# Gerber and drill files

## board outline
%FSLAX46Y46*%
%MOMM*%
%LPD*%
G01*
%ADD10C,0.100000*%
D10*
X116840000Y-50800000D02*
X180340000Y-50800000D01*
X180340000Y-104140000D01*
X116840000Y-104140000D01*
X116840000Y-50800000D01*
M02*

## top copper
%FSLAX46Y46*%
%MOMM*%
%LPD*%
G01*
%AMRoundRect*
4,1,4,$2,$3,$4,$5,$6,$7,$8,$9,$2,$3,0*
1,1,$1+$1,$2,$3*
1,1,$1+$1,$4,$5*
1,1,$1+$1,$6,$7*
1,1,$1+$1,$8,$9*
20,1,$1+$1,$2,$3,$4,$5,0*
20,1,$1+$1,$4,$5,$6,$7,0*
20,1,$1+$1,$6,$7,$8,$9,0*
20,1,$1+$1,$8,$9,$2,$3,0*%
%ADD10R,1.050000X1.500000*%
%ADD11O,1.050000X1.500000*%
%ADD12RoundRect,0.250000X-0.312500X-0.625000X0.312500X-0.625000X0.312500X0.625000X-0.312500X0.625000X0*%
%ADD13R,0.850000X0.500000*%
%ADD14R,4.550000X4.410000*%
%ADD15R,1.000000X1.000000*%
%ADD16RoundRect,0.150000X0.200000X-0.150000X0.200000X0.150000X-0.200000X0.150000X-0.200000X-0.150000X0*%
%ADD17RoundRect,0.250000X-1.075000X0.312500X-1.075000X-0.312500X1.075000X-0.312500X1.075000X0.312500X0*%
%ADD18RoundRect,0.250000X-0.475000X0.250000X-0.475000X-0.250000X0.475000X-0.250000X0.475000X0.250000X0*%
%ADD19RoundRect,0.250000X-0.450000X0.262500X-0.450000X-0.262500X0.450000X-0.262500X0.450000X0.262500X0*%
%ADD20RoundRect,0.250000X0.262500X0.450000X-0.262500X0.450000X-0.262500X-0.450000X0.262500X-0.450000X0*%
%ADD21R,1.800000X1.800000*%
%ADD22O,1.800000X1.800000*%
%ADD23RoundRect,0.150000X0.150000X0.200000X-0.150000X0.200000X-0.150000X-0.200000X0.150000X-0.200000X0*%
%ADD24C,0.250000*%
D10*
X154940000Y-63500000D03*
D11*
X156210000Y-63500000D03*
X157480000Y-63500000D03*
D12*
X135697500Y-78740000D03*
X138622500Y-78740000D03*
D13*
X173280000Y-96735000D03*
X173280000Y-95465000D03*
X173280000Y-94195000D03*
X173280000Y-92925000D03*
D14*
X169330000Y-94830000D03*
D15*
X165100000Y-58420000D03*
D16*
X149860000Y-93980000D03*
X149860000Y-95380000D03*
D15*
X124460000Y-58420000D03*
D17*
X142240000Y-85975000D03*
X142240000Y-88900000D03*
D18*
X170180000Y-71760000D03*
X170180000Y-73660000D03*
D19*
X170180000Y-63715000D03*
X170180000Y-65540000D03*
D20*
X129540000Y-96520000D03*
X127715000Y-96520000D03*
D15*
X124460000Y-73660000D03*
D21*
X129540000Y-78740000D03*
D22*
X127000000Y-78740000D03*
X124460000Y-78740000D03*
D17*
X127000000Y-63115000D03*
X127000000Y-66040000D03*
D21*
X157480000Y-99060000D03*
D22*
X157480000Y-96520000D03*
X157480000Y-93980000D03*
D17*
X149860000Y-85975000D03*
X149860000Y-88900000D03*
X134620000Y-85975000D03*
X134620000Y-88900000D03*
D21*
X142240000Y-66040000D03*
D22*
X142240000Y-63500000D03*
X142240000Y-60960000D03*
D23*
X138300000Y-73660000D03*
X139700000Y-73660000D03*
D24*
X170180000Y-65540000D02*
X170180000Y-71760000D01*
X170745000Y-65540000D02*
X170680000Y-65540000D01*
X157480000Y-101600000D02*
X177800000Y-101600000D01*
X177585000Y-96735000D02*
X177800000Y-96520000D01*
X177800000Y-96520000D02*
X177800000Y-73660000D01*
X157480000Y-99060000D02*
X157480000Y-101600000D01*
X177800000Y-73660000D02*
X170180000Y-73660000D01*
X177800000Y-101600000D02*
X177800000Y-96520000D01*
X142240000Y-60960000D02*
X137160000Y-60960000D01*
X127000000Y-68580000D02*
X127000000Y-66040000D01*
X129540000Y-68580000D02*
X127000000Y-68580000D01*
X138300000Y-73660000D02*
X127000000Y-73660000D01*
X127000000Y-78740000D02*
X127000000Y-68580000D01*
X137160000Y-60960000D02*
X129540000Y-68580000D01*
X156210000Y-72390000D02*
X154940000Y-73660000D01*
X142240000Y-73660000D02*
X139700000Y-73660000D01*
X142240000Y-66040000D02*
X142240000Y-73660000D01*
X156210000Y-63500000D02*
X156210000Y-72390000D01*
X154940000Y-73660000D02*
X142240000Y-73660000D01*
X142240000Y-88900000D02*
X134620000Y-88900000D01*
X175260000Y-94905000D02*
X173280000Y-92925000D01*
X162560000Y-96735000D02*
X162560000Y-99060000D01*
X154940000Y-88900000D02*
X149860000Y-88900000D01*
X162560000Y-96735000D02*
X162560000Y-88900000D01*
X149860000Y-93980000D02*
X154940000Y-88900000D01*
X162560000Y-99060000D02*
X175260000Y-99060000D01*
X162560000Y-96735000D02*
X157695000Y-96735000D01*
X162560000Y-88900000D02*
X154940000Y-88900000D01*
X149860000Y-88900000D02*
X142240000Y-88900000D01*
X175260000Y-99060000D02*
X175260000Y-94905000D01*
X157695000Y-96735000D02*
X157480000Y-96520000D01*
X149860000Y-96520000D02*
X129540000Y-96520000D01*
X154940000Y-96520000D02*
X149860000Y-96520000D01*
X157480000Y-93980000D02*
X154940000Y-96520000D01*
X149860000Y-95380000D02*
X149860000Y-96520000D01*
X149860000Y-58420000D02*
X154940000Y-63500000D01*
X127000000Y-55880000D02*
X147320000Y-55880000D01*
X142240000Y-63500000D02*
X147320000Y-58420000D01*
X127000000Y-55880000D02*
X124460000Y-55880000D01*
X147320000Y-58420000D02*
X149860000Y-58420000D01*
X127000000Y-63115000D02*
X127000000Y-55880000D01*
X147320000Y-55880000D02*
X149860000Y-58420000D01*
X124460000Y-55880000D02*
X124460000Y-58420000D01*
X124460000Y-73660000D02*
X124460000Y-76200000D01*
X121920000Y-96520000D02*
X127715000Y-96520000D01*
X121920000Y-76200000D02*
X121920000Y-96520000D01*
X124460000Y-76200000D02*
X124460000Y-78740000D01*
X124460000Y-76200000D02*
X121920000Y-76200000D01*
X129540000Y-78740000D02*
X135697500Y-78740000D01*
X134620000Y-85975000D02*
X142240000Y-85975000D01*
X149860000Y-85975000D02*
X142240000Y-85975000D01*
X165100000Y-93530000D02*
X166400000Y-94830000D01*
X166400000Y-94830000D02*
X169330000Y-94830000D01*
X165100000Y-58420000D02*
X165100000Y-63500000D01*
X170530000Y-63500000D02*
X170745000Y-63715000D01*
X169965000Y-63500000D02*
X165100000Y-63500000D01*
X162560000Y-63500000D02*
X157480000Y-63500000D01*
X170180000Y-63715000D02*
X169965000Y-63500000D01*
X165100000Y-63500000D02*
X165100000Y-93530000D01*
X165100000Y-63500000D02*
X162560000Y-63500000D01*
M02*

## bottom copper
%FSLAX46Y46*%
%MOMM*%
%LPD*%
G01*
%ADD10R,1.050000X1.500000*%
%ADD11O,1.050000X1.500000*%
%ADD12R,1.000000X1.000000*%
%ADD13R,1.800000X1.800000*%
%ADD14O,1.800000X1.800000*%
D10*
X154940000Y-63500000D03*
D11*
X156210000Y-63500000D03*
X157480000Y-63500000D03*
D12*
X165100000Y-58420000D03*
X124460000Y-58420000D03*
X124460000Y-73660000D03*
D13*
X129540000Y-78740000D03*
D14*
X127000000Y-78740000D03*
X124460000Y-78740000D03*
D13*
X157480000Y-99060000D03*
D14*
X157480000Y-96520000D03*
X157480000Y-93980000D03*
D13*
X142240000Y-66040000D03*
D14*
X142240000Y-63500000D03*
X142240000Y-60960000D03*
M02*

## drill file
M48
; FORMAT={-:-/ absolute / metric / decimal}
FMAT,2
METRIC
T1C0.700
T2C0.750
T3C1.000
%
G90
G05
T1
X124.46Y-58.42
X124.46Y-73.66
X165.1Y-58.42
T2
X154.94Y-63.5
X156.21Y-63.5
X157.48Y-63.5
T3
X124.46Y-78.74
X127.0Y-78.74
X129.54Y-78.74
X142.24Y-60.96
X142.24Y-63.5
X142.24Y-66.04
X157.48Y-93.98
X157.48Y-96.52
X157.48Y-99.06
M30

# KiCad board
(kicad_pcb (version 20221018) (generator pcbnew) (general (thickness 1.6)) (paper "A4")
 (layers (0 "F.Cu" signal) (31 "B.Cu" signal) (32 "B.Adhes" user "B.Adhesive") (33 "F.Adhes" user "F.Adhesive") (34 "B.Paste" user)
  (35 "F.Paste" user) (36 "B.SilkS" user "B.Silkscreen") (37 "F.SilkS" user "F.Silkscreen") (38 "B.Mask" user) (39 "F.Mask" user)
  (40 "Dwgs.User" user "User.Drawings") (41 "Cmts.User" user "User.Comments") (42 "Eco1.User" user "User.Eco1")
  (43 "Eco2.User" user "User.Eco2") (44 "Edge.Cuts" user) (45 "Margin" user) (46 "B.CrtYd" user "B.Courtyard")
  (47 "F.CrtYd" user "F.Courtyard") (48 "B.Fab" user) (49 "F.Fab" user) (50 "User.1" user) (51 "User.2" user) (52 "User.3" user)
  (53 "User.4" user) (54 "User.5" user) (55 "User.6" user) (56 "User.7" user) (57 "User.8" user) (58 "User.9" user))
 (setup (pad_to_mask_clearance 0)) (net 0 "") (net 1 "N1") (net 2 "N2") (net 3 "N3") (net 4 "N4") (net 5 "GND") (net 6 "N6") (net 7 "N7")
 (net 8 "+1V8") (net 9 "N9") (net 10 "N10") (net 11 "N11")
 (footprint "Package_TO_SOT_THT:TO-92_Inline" (layer "F.Cu") (at 154.94 63.5)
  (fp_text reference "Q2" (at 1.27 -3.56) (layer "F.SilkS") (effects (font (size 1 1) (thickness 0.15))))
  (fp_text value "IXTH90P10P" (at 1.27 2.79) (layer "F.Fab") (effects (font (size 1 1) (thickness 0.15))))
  (pad "1" thru_hole rect (at 0 0) (size 1.05 1.5) (drill 0.75) (layers "*.Cu" "*.Mask") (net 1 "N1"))
  (pad "2" thru_hole oval (at 1.27 0) (size 1.05 1.5) (drill 0.75) (layers "*.Cu" "*.Mask") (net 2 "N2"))
  (pad "3" thru_hole oval (at 2.54 0) (size 1.05 1.5) (drill 0.75) (layers "*.Cu" "*.Mask") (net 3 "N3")))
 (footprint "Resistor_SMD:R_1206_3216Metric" (layer "F.Cu") (at 137.16 78.74)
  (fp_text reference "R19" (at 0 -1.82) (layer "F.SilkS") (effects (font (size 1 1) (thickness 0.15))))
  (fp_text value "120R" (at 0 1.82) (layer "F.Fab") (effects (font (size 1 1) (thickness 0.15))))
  (pad "1" smd roundrect (at -1.4625 0) (size 1.125 1.75) (layers "F.Cu" "F.Paste" "F.Mask") (roundrect_rratio 0.222222) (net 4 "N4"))
  (pad "2" smd roundrect (at 1.4625 0) (size 1.125 1.75) (layers "F.Cu" "F.Paste" "F.Mask") (roundrect_rratio 0.222222) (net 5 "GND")))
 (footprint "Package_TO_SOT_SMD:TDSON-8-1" (layer "F.Cu") (at 170.38 94.83 180)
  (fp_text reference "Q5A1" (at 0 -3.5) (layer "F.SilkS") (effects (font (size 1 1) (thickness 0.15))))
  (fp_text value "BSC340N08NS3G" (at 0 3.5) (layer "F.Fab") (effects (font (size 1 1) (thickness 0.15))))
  (pad "" smd rect (at -0.2 -0.85 180) (size 1.5 1.5) (layers "F.Paste"))
  (pad "" smd rect (at -0.2 0.85 180) (size 1.5 1.5) (layers "F.Paste"))
  (pad "" smd custom (at 0.65 0 180) (size 3.75 4.41) (layers "F.Mask") (zone_connect 0) (thermal_bridge_angle 45)
   (options (clearance outline) (anchor rect)) (primitives))
  (pad "" smd rect (at 1.5 -0.85 180) (size 1.5 1.5) (layers "F.Paste"))
  (pad "" smd rect (at 1.5 0.85 180) (size 1.5 1.5) (layers "F.Paste"))
  (pad "" smd rect (at 2.905 -1.905 180) (size 0.75 0.5) (layers "F.Paste"))
  (pad "" smd rect (at 2.905 -0.635 180) (size 0.75 0.5) (layers "F.Paste"))
  (pad "" smd rect (at 2.905 0.635 180) (size 0.75 0.5) (layers "F.Paste"))
  (pad "" smd rect (at 2.905 1.905 180) (size 0.75 0.5) (layers "F.Paste"))
  (pad "1" smd rect (at -2.9 -1.905 180) (size 0.85 0.5) (layers "F.Cu" "F.Paste" "F.Mask") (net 5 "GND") (solder_paste_margin -0.05))
  (pad "2" smd rect (at -2.9 -0.635 180) (size 0.85 0.5) (layers "F.Cu" "F.Paste" "F.Mask") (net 5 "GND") (solder_paste_margin -0.05))
  (pad "3" smd rect (at -2.9 0.635 180) (size 0.85 0.5) (layers "F.Cu" "F.Paste" "F.Mask") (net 5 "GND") (solder_paste_margin -0.05))
  (pad "4" smd rect (at -2.9 1.905 180) (size 0.85 0.5) (layers "F.Cu" "F.Paste" "F.Mask") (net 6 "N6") (solder_paste_margin -0.05))
  (pad "5" smd rect (at 1.05 0 180) (size 4.55 4.41) (layers "F.Cu") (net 3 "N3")))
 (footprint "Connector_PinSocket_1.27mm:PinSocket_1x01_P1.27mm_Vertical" (layer "F.Cu") (at 165.1 58.42)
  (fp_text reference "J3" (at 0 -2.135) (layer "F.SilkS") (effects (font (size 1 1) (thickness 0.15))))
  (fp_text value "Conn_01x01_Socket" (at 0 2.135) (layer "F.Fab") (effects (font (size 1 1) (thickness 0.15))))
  (pad "1" thru_hole rect (at 0 0) (size 1 1) (drill 0.7) (layers "*.Cu" "*.Mask") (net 3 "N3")))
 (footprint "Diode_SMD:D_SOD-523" (layer "F.Cu") (at 149.86 94.68 -90)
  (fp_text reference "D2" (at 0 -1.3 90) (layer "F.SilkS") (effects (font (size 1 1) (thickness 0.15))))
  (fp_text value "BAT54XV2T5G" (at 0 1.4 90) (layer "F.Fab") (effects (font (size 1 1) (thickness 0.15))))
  (pad "1" smd roundrect (at -0.7 0 90) (size 0.6 0.7) (layers "F.Cu" "F.Paste" "F.Mask") (roundrect_rratio 0.25) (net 6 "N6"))
  (pad "2" smd roundrect (at 0.7 0 90) (size 0.6 0.7) (layers "F.Cu" "F.Paste" "F.Mask") (roundrect_rratio 0.25) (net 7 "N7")))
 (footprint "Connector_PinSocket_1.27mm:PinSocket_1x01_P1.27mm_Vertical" (layer "F.Cu") (at 124.46 58.42)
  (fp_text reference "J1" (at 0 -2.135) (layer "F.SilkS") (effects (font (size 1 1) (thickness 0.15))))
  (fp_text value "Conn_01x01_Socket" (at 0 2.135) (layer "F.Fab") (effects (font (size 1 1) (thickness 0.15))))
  (pad "1" thru_hole rect (at 0 0) (size 1 1) (drill 0.7) (layers "*.Cu" "*.Mask") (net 1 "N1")))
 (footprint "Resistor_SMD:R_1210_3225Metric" (layer "F.Cu") (at 142.24 87.4375 -90)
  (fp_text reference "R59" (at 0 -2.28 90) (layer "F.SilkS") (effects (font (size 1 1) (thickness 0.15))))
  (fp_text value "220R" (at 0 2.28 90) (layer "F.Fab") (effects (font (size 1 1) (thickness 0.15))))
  (pad "1" smd roundrect (at -1.4625 0 270) (size 1.125 2.65) (layers "F.Cu" "F.Paste" "F.Mask") (roundrect_rratio 0.222222) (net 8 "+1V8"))
  (pad "2" smd roundrect (at 1.4625 0 270) (size 1.125 2.65) (layers "F.Cu" "F.Paste" "F.Mask") (roundrect_rratio 0.222222) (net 6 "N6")))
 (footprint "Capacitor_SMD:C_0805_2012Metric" (layer "F.Cu") (at 170.18 72.71 -90)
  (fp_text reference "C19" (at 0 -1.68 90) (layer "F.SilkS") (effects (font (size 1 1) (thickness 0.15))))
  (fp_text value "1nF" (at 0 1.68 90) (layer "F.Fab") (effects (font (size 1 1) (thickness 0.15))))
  (pad "1" smd roundrect (at -0.95 0 270) (size 1 1.45) (layers "F.Cu" "F.Paste" "F.Mask") (roundrect_rratio 0.25) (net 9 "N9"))
  (pad "2" smd roundrect (at 0.95 0 270) (size 1 1.45) (layers "F.Cu" "F.Paste" "F.Mask") (roundrect_rratio 0.25) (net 5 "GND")))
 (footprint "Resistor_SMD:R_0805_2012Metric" (layer "F.Cu") (at 170.18 64.6275 -90)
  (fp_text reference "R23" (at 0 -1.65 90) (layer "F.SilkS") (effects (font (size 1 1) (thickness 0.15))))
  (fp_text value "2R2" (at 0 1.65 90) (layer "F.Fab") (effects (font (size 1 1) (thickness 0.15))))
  (pad "1" smd roundrect (at -0.9125 0 270) (size 1.025 1.4) (layers "F.Cu" "F.Paste" "F.Mask") (roundrect_rratio 0.243902) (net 3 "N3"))
  (pad "2" smd roundrect (at 0.9125 0 270) (size 1.025 1.4) (layers "F.Cu" "F.Paste" "F.Mask") (roundrect_rratio 0.243902) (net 9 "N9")))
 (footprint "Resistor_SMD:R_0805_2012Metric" (layer "F.Cu") (at 128.6275 96.52 180)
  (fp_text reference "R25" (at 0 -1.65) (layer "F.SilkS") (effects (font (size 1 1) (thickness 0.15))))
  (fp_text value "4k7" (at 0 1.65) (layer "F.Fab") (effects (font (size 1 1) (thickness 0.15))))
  (pad "1" smd roundrect (at -0.9125 0 180) (size 1.025 1.4) (layers "F.Cu" "F.Paste" "F.Mask") (roundrect_rratio 0.243902) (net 7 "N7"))
  (pad "2" smd roundrect (at 0.9125 0 180) (size 1.025 1.4) (layers "F.Cu" "F.Paste" "F.Mask") (roundrect_rratio 0.243902) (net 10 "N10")))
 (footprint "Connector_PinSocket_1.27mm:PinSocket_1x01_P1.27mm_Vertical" (layer "F.Cu") (at 124.46 73.66)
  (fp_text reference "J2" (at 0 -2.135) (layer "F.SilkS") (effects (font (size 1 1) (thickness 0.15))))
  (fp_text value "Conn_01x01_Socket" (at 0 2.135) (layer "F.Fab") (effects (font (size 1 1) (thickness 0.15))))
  (pad "1" thru_hole rect (at 0 0) (size 1 1) (drill 0.7) (layers "*.Cu" "*.Mask") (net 10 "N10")))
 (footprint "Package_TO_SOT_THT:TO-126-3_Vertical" (layer "F.Cu") (at 129.54 78.74 180)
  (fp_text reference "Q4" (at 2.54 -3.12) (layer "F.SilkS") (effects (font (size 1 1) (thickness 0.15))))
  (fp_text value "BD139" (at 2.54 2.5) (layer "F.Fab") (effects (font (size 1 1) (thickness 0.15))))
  (pad "1" thru_hole rect (at 0 0 180) (size 1.8 1.8) (drill 1) (layers "*.Cu" "*.Mask") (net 4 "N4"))
  (pad "2" thru_hole oval (at 2.54 0 180) (size 1.8 1.8) (drill 1) (layers "*.Cu" "*.Mask") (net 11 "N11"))
  (pad "3" thru_hole oval (at 5.08 0 180) (size 1.8 1.8) (drill 1) (layers "*.Cu" "*.Mask") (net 10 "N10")))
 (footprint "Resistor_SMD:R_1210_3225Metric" (layer "F.Cu") (at 127 64.5775 -90)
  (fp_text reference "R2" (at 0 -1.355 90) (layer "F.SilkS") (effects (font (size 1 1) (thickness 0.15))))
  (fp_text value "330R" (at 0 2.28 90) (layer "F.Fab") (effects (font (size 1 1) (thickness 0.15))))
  (pad "1" smd roundrect (at -1.4625 0 270) (size 1.125 2.65) (layers "F.Cu" "F.Paste" "F.Mask") (roundrect_rratio 0.222222) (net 1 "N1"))
  (pad "2" smd roundrect (at 1.4625 0 270) (size 1.125 2.65) (layers "F.Cu" "F.Paste" "F.Mask") (roundrect_rratio 0.222222) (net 11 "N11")))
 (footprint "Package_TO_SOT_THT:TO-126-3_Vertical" (layer "F.Cu") (at 157.48 99.06 90)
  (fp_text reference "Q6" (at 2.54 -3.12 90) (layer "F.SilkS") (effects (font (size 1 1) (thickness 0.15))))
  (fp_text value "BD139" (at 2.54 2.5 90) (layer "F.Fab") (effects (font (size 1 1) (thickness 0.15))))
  (pad "1" thru_hole rect (at 0 0 90) (size 1.8 1.8) (drill 1) (layers "*.Cu" "*.Mask") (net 5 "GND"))
  (pad "2" thru_hole oval (at 2.54 0 90) (size 1.8 1.8) (drill 1) (layers "*.Cu" "*.Mask") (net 6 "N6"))
  (pad "3" thru_hole oval (at 5.08 0 90) (size 1.8 1.8) (drill 1) (layers "*.Cu" "*.Mask") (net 7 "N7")))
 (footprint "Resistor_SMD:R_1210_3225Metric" (layer "F.Cu") (at 149.86 87.4375 -90)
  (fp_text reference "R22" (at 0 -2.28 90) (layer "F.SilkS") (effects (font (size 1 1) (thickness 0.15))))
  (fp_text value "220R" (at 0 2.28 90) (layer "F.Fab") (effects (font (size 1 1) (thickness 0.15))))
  (pad "1" smd roundrect (at -1.4625 0 270) (size 1.125 2.65) (layers "F.Cu" "F.Paste" "F.Mask") (roundrect_rratio 0.222222) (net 8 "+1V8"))
  (pad "2" smd roundrect (at 1.4625 0 270) (size 1.125 2.65) (layers "F.Cu" "F.Paste" "F.Mask") (roundrect_rratio 0.222222) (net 6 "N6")))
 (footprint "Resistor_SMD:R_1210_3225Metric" (layer "F.Cu") (at 134.62 87.4375 -90)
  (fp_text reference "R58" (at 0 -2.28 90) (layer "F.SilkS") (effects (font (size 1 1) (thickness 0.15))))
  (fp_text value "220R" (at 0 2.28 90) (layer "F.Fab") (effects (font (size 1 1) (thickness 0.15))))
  (pad "1" smd roundrect (at -1.4625 0 270) (size 1.125 2.65) (layers "F.Cu" "F.Paste" "F.Mask") (roundrect_rratio 0.222222) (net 8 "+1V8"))
  (pad "2" smd roundrect (at 1.4625 0 270) (size 1.125 2.65) (layers "F.Cu" "F.Paste" "F.Mask") (roundrect_rratio 0.222222) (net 6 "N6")))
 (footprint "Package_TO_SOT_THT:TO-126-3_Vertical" (layer "F.Cu") (at 142.24 66.04 90)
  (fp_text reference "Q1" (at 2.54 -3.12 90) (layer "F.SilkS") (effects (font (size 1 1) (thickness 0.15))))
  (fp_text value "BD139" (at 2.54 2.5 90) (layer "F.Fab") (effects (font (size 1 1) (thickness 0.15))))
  (pad "1" thru_hole rect (at 0 0 90) (size 1.8 1.8) (drill 1) (layers "*.Cu" "*.Mask") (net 2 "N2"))
  (pad "2" thru_hole oval (at 2.54 0 90) (size 1.8 1.8) (drill 1) (layers "*.Cu" "*.Mask") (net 1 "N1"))
  (pad "3" thru_hole oval (at 5.08 0 90) (size 1.8 1.8) (drill 1) (layers "*.Cu" "*.Mask") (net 11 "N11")))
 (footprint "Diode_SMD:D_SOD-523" (layer "F.Cu") (at 139 73.66)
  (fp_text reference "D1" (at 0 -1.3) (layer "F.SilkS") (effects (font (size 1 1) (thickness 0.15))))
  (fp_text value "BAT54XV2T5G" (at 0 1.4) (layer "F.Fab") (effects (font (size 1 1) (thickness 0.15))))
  (pad "1" smd roundrect (at -0.7 0 180) (size 0.6 0.7) (layers "F.Cu" "F.Paste" "F.Mask") (roundrect_rratio 0.25) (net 11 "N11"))
  (pad "2" smd roundrect (at 0.7 0 180) (size 0.6 0.7) (layers "F.Cu" "F.Paste" "F.Mask") (roundrect_rratio 0.25) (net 2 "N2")))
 (gr_poly
  (pts (xy 116.84 50.8) (xy 180.34 50.8) (xy 180.34 104.14) (xy 116.84 104.14)) (stroke (width 0.1) (type solid)) (fill none)
  (layer "Edge.Cuts"))
 (segment (start 170.18 65.54) (end 170.18 71.76) (width 0.25) (layer "F.Cu") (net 9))
 (segment (start 170.745 65.54) (end 170.68 65.54) (width 0.25) (layer "F.Cu") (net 9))
 (segment (start 157.48 101.6) (end 177.8 101.6) (width 0.25) (layer "F.Cu") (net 5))
 (segment (start 177.585 96.735) (end 177.8 96.52) (width 0.25) (layer "F.Cu") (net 5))
 (segment (start 177.8 96.52) (end 177.8 73.66) (width 0.25) (layer "F.Cu") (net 5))
 (segment (start 157.48 99.06) (end 157.48 101.6) (width 0.25) (layer "F.Cu") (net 5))
 (segment (start 177.8 73.66) (end 170.18 73.66) (width 0.25) (layer "F.Cu") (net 5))
 (segment (start 177.8 101.6) (end 177.8 96.52) (width 0.25) (layer "F.Cu") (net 5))
 (segment (start 142.24 60.96) (end 137.16 60.96) (width 0.25) (layer "F.Cu") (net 11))
 (segment (start 127 68.58) (end 127 66.04) (width 0.25) (layer "F.Cu") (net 11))
 (segment (start 129.54 68.58) (end 127 68.58) (width 0.25) (layer "F.Cu") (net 11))
 (segment (start 138.3 73.66) (end 127 73.66) (width 0.25) (layer "F.Cu") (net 11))
 (segment (start 127 78.74) (end 127 68.58) (width 0.25) (layer "F.Cu") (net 11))
 (segment (start 137.16 60.96) (end 129.54 68.58) (width 0.25) (layer "F.Cu") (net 11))
 (segment (start 156.21 72.39) (end 154.94 73.66) (width 0.25) (layer "F.Cu") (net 2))
 (segment (start 142.24 73.66) (end 139.7 73.66) (width 0.25) (layer "F.Cu") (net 2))
 (segment (start 142.24 66.04) (end 142.24 73.66) (width 0.25) (layer "F.Cu") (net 2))
 (segment (start 156.21 63.5) (end 156.21 72.39) (width 0.25) (layer "F.Cu") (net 2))
 (segment (start 154.94 73.66) (end 142.24 73.66) (width 0.25) (layer "F.Cu") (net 2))
 (segment (start 142.24 88.9) (end 134.62 88.9) (width 0.25) (layer "F.Cu") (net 6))
 (segment (start 175.26 94.905) (end 173.28 92.925) (width 0.25) (layer "F.Cu") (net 6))
 (segment (start 162.56 96.735) (end 162.56 99.06) (width 0.25) (layer "F.Cu") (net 6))
 (segment (start 154.94 88.9) (end 149.86 88.9) (width 0.25) (layer "F.Cu") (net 6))
 (segment (start 162.56 96.735) (end 162.56 88.9) (width 0.25) (layer "F.Cu") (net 6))
 (segment (start 149.86 93.98) (end 154.94 88.9) (width 0.25) (layer "F.Cu") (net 6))
 (segment (start 162.56 99.06) (end 175.26 99.06) (width 0.25) (layer "F.Cu") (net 6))
 (segment (start 162.56 96.735) (end 157.695 96.735) (width 0.25) (layer "F.Cu") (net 6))
 (segment (start 162.56 88.9) (end 154.94 88.9) (width 0.25) (layer "F.Cu") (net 6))
 (segment (start 149.86 88.9) (end 142.24 88.9) (width 0.25) (layer "F.Cu") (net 6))
 (segment (start 175.26 99.06) (end 175.26 94.905) (width 0.25) (layer "F.Cu") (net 6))
 (segment (start 157.695 96.735) (end 157.48 96.52) (width 0.25) (layer "F.Cu") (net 6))
 (segment (start 149.86 96.52) (end 129.54 96.52) (width 0.25) (layer "F.Cu") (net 7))
 (segment (start 154.94 96.52) (end 149.86 96.52) (width 0.25) (layer "F.Cu") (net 7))
 (segment (start 157.48 93.98) (end 154.94 96.52) (width 0.25) (layer "F.Cu") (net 7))
 (segment (start 149.86 95.38) (end 149.86 96.52) (width 0.25) (layer "F.Cu") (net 7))
 (segment (start 149.86 58.42) (end 154.94 63.5) (width 0.25) (layer "F.Cu") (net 1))
 (segment (start 127 55.88) (end 147.32 55.88) (width 0.25) (layer "F.Cu") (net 1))
 (segment (start 142.24 63.5) (end 147.32 58.42) (width 0.25) (layer "F.Cu") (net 1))
 (segment (start 127 55.88) (end 124.46 55.88) (width 0.25) (layer "F.Cu") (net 1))
 (segment (start 147.32 58.42) (end 149.86 58.42) (width 0.25) (layer "F.Cu") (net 1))
 (segment (start 127 63.115) (end 127 55.88) (width 0.25) (layer "F.Cu") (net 1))
 (segment (start 147.32 55.88) (end 149.86 58.42) (width 0.25) (layer "F.Cu") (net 1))
 (segment (start 124.46 55.88) (end 124.46 58.42) (width 0.25) (layer "F.Cu") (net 1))
 (segment (start 124.46 73.66) (end 124.46 76.2) (width 0.25) (layer "F.Cu") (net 10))
 (segment (start 121.92 96.52) (end 127.715 96.52) (width 0.25) (layer "F.Cu") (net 10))
 (segment (start 121.92 76.2) (end 121.92 96.52) (width 0.25) (layer "F.Cu") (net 10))
 (segment (start 124.46 76.2) (end 124.46 78.74) (width 0.25) (layer "F.Cu") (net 10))
 (segment (start 124.46 76.2) (end 121.92 76.2) (width 0.25) (layer "F.Cu") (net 10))
 (segment (start 129.54 78.74) (end 135.6975 78.74) (width 0.25) (layer "F.Cu") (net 4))
 (segment (start 134.62 85.975) (end 142.24 85.975) (width 0.25) (layer "F.Cu") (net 8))
 (segment (start 149.86 85.975) (end 142.24 85.975) (width 0.25) (layer "F.Cu") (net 8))
 (segment (start 165.1 93.53) (end 166.4 94.83) (width 0.25) (layer "F.Cu") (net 3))
 (segment (start 166.4 94.83) (end 169.33 94.83) (width 0.25) (layer "F.Cu") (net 3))
 (segment (start 165.1 58.42) (end 165.1 63.5) (width 0.25) (layer "F.Cu") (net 3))
 (segment (start 170.53 63.5) (end 170.745 63.715) (width 0.25) (layer "F.Cu") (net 3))
 (segment (start 169.965 63.5) (end 165.1 63.5) (width 0.25) (layer "F.Cu") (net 3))
 (segment (start 162.56 63.5) (end 157.48 63.5) (width 0.25) (layer "F.Cu") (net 3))
 (segment (start 170.18 63.715) (end 169.965 63.5) (width 0.25) (layer "F.Cu") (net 3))
 (segment (start 165.1 63.5) (end 165.1 93.53) (width 0.25) (layer "F.Cu") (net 3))
 (segment (start 165.1 63.5) (end 162.56 63.5) (width 0.25) (layer "F.Cu") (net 3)))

